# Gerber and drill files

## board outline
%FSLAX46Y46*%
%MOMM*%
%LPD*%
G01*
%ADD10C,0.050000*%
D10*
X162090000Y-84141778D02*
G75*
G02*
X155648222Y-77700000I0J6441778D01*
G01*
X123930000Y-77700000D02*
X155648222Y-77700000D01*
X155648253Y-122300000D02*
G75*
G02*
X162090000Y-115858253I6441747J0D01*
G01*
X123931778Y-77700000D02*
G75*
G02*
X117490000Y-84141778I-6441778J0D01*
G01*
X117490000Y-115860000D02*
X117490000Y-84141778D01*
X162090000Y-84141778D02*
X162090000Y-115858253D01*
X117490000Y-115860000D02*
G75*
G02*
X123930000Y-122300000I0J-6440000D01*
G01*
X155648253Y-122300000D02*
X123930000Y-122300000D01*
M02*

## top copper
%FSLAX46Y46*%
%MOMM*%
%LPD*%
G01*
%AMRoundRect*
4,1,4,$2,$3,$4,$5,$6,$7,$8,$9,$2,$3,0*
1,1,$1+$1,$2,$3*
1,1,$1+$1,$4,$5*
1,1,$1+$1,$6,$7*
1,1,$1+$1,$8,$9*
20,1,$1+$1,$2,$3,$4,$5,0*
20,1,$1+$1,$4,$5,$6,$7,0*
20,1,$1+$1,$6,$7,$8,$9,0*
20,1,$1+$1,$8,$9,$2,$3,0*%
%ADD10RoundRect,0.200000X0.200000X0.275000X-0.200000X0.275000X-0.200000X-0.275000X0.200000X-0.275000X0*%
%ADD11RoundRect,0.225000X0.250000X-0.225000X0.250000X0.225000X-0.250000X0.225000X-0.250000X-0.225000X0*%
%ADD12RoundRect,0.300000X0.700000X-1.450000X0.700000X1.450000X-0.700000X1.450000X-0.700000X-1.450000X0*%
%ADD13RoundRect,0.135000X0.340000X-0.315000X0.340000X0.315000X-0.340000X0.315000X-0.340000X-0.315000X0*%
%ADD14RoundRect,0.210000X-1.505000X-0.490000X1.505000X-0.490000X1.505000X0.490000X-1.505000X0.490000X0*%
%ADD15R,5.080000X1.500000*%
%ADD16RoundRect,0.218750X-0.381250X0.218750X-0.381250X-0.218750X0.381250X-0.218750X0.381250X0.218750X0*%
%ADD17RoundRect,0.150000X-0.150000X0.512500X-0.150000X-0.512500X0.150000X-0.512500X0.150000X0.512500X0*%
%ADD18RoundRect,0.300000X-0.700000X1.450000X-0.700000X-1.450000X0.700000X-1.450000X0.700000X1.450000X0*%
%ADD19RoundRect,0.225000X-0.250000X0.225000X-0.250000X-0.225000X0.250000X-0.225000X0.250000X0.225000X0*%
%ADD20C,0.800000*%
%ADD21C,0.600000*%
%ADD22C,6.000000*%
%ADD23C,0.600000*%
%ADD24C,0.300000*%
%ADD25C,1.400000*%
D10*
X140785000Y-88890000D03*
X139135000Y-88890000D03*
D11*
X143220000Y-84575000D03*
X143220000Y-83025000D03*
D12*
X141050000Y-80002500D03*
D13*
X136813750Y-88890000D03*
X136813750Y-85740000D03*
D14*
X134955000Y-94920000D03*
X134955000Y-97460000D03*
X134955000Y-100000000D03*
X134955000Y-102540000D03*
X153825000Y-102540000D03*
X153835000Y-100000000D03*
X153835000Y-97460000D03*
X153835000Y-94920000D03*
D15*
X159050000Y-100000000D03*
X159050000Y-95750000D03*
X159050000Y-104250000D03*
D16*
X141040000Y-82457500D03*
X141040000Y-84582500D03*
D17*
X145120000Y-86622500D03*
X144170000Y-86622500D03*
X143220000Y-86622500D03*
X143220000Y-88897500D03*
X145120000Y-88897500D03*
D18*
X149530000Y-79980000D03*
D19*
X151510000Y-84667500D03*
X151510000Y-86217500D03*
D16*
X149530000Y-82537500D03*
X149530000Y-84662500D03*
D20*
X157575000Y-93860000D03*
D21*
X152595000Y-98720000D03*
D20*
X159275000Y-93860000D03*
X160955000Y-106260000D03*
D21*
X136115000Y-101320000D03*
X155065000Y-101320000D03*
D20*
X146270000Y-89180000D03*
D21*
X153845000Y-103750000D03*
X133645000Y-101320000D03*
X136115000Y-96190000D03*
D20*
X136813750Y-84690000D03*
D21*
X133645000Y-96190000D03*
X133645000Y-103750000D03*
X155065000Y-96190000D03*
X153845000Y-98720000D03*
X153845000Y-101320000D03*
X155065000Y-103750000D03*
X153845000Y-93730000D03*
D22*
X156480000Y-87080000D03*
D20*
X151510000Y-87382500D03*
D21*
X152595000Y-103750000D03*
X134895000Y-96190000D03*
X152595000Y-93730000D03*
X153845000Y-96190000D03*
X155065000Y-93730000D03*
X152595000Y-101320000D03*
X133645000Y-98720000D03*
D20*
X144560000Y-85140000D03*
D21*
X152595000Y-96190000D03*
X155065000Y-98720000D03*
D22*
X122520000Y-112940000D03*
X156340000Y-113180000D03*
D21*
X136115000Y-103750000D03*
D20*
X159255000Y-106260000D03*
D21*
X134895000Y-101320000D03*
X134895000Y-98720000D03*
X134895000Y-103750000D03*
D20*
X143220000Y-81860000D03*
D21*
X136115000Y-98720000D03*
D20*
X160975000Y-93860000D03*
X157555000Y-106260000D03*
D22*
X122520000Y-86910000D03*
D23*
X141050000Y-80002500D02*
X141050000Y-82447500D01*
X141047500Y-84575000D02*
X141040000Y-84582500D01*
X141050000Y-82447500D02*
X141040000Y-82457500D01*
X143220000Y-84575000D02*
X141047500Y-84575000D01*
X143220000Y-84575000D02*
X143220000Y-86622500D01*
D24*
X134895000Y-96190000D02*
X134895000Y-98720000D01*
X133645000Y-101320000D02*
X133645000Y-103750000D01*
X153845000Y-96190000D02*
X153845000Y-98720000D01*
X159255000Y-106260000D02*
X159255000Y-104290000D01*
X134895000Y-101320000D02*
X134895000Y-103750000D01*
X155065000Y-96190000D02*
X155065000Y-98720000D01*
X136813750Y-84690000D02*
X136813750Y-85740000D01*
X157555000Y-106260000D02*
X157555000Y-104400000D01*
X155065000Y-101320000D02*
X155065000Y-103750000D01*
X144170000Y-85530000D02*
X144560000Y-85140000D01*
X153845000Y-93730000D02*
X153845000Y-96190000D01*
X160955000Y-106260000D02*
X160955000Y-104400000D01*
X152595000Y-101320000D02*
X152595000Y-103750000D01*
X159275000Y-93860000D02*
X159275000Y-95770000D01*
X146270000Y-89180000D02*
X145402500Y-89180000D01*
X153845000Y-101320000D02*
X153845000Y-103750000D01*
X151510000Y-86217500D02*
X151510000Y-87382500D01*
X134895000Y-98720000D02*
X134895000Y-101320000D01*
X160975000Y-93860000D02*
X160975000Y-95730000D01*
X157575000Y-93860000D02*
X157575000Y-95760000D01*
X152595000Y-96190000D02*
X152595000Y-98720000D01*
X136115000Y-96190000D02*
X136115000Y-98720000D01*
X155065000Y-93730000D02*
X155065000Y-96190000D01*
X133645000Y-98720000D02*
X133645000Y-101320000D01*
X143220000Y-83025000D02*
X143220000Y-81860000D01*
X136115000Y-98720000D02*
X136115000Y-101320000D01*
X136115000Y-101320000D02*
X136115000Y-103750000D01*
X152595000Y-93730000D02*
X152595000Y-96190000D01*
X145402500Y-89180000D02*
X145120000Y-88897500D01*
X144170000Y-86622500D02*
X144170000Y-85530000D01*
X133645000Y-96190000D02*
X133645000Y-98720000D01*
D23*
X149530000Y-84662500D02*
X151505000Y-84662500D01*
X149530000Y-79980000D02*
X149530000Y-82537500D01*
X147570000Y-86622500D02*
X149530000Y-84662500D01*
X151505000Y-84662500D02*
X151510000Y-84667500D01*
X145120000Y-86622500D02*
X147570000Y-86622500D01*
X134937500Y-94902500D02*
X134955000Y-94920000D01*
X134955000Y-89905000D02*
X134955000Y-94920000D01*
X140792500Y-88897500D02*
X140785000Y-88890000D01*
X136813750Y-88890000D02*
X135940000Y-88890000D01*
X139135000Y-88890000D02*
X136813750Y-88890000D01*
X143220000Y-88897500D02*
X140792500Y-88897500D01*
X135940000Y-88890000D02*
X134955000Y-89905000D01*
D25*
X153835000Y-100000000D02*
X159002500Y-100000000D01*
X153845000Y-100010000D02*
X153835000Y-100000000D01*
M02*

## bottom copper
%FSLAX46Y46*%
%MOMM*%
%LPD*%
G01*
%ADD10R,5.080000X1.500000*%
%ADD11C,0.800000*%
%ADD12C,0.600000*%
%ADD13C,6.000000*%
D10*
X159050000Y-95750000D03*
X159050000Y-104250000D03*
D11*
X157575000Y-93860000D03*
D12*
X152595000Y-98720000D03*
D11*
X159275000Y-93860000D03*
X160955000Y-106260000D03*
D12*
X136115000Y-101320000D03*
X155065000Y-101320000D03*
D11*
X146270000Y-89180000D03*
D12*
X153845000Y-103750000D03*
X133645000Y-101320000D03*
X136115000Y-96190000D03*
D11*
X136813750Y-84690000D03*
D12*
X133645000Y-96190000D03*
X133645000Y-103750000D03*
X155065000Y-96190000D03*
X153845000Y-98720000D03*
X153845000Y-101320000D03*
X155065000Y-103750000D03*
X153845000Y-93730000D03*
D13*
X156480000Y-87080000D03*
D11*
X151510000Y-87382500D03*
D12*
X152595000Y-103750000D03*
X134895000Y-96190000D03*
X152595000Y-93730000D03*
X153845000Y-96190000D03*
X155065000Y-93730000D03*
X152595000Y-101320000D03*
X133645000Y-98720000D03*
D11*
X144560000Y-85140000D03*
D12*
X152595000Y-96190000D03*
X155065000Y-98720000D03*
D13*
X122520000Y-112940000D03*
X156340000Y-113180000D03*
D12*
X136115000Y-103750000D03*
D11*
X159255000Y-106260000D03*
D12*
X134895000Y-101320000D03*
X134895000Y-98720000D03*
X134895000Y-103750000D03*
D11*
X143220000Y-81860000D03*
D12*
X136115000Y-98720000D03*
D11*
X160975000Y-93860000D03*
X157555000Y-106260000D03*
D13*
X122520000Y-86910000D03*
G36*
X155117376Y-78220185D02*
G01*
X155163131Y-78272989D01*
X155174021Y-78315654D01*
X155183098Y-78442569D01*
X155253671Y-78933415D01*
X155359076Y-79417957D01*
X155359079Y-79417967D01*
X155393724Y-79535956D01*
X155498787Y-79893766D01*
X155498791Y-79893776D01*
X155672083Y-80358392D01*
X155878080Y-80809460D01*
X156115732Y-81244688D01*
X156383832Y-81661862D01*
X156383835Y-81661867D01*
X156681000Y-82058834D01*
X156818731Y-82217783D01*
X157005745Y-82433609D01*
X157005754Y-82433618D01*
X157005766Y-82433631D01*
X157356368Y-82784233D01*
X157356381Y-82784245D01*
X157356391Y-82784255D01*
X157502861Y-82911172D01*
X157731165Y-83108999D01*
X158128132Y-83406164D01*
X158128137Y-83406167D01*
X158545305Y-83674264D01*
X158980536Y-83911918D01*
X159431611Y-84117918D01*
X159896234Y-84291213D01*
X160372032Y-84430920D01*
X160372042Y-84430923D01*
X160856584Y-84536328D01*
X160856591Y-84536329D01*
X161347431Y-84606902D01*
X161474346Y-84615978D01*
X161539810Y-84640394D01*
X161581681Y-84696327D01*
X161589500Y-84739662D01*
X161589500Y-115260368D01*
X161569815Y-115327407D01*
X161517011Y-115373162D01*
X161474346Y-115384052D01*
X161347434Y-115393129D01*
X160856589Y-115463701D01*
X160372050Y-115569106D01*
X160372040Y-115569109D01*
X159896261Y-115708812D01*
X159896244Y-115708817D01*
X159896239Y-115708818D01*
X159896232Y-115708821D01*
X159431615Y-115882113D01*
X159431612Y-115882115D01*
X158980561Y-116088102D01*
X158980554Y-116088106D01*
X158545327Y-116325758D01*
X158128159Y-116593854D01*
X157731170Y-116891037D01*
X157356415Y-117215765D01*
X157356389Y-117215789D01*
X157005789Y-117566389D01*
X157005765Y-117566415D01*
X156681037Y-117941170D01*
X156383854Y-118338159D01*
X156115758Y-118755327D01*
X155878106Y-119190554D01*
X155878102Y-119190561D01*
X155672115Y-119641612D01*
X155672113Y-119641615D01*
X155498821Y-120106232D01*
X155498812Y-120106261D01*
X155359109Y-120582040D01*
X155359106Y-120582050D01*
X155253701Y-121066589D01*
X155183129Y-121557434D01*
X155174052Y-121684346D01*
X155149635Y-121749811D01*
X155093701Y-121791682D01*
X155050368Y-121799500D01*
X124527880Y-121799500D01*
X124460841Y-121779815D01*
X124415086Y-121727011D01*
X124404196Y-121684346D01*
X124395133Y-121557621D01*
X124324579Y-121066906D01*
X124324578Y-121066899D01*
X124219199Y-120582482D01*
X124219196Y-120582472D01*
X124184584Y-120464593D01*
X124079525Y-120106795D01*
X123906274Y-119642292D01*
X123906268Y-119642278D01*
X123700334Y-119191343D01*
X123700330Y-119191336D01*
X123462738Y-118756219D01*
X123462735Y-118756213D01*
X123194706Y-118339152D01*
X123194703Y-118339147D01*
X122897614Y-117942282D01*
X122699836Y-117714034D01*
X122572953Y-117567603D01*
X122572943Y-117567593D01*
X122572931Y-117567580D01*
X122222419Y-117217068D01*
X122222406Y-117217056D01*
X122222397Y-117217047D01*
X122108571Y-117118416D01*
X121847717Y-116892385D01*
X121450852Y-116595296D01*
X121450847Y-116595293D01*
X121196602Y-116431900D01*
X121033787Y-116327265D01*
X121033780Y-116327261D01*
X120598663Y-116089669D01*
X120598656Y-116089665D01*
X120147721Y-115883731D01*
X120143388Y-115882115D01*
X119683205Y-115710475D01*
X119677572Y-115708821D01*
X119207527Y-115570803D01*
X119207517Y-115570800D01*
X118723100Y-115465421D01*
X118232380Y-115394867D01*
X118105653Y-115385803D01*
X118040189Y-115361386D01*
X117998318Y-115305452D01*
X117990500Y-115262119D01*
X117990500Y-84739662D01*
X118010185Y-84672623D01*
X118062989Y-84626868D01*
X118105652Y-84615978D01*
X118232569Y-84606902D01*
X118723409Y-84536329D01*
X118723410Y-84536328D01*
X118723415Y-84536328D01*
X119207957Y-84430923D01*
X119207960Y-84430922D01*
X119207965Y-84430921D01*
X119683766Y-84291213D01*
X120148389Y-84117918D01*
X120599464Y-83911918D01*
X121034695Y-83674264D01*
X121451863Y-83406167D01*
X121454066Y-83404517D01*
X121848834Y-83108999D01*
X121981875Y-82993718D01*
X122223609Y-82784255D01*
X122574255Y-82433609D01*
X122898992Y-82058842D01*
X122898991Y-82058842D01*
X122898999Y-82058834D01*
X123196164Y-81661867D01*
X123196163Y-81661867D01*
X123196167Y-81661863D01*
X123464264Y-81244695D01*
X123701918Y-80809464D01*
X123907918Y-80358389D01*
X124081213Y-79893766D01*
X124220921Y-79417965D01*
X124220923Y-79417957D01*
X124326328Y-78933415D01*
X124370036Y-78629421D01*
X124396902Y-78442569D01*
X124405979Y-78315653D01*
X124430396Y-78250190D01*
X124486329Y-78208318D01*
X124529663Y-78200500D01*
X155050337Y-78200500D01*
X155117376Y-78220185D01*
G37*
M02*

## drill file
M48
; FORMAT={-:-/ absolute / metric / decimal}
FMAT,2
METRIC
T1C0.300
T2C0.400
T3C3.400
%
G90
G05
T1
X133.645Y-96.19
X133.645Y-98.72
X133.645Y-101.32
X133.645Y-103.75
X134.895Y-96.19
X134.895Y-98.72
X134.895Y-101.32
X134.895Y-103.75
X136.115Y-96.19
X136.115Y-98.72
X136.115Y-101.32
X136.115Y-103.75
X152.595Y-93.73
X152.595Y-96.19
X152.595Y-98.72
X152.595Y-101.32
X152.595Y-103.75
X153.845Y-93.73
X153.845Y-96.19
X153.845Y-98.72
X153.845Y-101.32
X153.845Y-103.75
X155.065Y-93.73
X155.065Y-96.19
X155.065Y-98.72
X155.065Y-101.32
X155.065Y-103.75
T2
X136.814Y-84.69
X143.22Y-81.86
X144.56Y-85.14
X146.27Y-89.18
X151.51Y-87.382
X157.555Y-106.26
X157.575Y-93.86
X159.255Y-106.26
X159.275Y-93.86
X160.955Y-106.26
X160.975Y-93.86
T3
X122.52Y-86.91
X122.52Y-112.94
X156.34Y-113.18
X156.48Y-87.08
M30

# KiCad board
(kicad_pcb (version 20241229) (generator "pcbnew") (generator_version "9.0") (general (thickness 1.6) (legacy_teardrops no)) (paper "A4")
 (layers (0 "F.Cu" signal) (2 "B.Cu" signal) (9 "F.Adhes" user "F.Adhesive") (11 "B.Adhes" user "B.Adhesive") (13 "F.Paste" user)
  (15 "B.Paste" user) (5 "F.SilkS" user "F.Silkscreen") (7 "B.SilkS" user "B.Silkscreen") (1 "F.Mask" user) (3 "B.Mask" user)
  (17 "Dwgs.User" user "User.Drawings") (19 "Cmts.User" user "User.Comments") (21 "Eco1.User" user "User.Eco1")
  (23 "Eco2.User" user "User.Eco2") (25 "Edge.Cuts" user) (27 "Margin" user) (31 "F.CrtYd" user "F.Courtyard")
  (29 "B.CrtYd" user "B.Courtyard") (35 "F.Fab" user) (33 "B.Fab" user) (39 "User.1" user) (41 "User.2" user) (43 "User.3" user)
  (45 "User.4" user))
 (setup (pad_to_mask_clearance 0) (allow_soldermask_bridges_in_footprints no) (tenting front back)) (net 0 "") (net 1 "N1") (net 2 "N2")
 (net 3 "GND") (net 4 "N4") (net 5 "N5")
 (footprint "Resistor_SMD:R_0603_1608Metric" (layer "F.Cu") (at 139.96 88.89 180)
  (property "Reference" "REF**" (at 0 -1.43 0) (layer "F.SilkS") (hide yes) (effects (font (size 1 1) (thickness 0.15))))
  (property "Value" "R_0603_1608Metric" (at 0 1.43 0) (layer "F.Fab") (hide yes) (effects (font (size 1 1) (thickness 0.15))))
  (pad "1" smd roundrect (at -0.825 0 180) (size 0.8 0.95) (layers "F.Cu" "F.Mask" "F.Paste") (roundrect_rratio 0.25) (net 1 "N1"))
  (pad "2" smd roundrect (at 0.825 0 180) (size 0.8 0.95) (layers "F.Cu" "F.Mask" "F.Paste") (roundrect_rratio 0.25) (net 1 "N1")))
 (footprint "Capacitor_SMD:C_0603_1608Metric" (layer "F.Cu") (at 143.22 83.8 90)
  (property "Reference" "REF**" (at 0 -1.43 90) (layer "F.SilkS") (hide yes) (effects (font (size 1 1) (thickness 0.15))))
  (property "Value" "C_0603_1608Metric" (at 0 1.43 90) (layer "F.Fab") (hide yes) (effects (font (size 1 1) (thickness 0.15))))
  (pad "1" smd roundrect (at -0.775 0 90) (size 0.9 0.95) (layers "F.Cu" "F.Mask" "F.Paste") (roundrect_rratio 0.25) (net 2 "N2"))
  (pad "2" smd roundrect (at 0.775 0 90) (size 0.9 0.95) (layers "F.Cu" "F.Mask" "F.Paste") (roundrect_rratio 0.25) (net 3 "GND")))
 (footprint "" (layer "F.Cu") (at 141.05 80.0125 180)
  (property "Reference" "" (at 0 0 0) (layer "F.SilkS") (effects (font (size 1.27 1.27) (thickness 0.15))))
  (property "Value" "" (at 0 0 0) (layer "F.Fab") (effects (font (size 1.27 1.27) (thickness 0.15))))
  (pad "3" smd roundrect (at 0 0.01 90) (size 3.5 2) (layers "F.Cu" "F.Mask" "F.Paste") (roundrect_rratio 0.15) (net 2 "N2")
   (thermal_bridge_angle 45)))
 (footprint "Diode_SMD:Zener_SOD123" (layer "F.Cu") (at 136.80375 88.89 90)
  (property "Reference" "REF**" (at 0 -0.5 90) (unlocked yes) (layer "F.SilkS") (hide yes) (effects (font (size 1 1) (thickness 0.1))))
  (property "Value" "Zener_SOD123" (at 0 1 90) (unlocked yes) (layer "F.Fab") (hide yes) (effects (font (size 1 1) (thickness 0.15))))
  (pad "1" smd roundrect (at 0 0.01 90) (size 0.9 0.95) (layers "F.Cu" "F.Mask" "F.Paste") (roundrect_rratio 0.15) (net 1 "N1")
   (thermal_bridge_angle 45))
  (pad "2" smd roundrect (at 3.15 0.01 90) (size 0.9 0.95) (layers "F.Cu" "F.Mask" "F.Paste") (roundrect_rratio 0.15) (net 3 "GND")
   (thermal_bridge_angle 45)))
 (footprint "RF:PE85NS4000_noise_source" (layer "F.Cu") (at 144.395 98.73)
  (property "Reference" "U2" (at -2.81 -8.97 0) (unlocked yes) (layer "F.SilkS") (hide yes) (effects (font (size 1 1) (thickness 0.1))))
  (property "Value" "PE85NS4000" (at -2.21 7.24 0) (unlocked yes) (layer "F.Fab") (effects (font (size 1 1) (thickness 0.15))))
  (pad "1" smd roundrect (at -9.44 -3.81) (size 3.43 1.4) (layers "F.Cu" "F.Mask" "F.Paste") (roundrect_rratio 0.15) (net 1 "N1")
   (thermal_bridge_angle 45))
  (pad "2" smd roundrect (at -9.44 -1.27) (size 3.43 1.4) (layers "F.Cu" "F.Mask" "F.Paste") (roundrect_rratio 0.15) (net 3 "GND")
   (thermal_bridge_angle 45))
  (pad "3" smd roundrect (at -9.44 1.27) (size 3.43 1.4) (layers "F.Cu" "F.Mask" "F.Paste") (roundrect_rratio 0.15) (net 3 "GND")
   (thermal_bridge_angle 45))
  (pad "4" smd roundrect (at -9.44 3.81) (size 3.43 1.4) (layers "F.Cu" "F.Mask" "F.Paste") (roundrect_rratio 0.15) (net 3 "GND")
   (thermal_bridge_angle 45))
  (pad "5" smd roundrect (at 9.43 3.81) (size 3.43 1.4) (layers "F.Cu" "F.Mask" "F.Paste") (roundrect_rratio 0.15) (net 3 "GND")
   (thermal_bridge_angle 45))
  (pad "6" smd roundrect (at 9.44 1.27) (size 3.43 1.4) (layers "F.Cu" "F.Mask" "F.Paste") (roundrect_rratio 0.15) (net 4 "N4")
   (thermal_bridge_angle 45))
  (pad "7" smd roundrect (at 9.44 -1.27) (size 3.43 1.4) (layers "F.Cu" "F.Mask" "F.Paste") (roundrect_rratio 0.15) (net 3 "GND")
   (thermal_bridge_angle 45))
  (pad "8" smd roundrect (at 9.44 -3.81) (size 3.43 1.4) (layers "F.Cu" "F.Mask" "F.Paste") (roundrect_rratio 0.15) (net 3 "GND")
   (thermal_bridge_angle 45)))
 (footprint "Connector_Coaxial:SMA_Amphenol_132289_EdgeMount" (layer "F.Cu") (at 159.05 100)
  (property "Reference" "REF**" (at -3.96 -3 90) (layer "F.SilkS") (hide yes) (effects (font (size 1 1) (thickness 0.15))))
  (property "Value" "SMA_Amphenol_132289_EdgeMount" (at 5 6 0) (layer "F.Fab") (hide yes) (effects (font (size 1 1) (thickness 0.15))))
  (pad "1" smd rect (at 0 0 90) (size 1.5 5.08) (layers "F.Cu" "F.Mask" "F.Paste") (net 4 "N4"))
  (pad "2" smd rect (at 0 -4.25 90) (size 1.5 5.08) (layers "F.Cu" "F.Mask" "F.Paste") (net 3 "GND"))
  (pad "2" smd rect (at 0 -4.25 90) (size 1.5 5.08) (layers "B.Cu" "B.Mask" "B.Paste") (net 3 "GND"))
  (pad "2" smd rect (at 0 4.25 90) (size 1.5 5.08) (layers "F.Cu" "F.Mask" "F.Paste") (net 3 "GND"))
  (pad "2" smd rect (at 0 4.25 90) (size 1.5 5.08) (layers "B.Cu" "B.Mask" "B.Paste") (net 3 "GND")))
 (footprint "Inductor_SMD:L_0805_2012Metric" (layer "F.Cu") (at 141.04 83.52 -90)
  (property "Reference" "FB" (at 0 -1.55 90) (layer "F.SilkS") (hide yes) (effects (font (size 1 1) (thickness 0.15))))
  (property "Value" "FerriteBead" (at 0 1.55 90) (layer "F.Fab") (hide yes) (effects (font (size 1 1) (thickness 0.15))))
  (pad "1" smd roundrect (at -1.0625 0 270) (size 0.875 1.2) (layers "F.Cu" "F.Mask" "F.Paste") (roundrect_rratio 0.25) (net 2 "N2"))
  (pad "2" smd roundrect (at 1.0625 0 270) (size 0.875 1.2) (layers "F.Cu" "F.Mask" "F.Paste") (roundrect_rratio 0.25) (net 2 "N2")))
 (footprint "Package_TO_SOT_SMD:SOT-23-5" (layer "F.Cu") (at 144.17 87.76 -90)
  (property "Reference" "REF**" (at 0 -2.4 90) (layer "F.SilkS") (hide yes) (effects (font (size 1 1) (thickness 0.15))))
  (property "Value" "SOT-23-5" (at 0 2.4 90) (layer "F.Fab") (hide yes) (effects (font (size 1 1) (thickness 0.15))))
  (pad "1" smd roundrect (at -1.1375 -0.95 270) (size 1.325 0.6) (layers "F.Cu" "F.Mask" "F.Paste") (roundrect_rratio 0.25) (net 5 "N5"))
  (pad "2" smd roundrect (at -1.1375 0 270) (size 1.325 0.6) (layers "F.Cu" "F.Mask" "F.Paste") (roundrect_rratio 0.25) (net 3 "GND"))
  (pad "3" smd roundrect (at -1.1375 0.95 270) (size 1.325 0.6) (layers "F.Cu" "F.Mask" "F.Paste") (roundrect_rratio 0.25) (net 2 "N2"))
  (pad "4" smd roundrect (at 1.1375 0.95 270) (size 1.325 0.6) (layers "F.Cu" "F.Mask" "F.Paste") (roundrect_rratio 0.25) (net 1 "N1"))
  (pad "5" smd roundrect (at 1.1375 -0.95 270) (size 1.325 0.6) (layers "F.Cu" "F.Mask" "F.Paste") (roundrect_rratio 0.25) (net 3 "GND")))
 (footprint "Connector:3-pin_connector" (layer "F.Cu") (at 149.53 79.98 -90)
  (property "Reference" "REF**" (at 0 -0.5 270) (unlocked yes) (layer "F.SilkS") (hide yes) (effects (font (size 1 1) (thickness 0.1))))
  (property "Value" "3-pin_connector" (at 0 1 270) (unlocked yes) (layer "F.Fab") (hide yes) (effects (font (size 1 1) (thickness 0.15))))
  (pad "1" smd roundrect (at 0 0 270) (size 3.5 2) (layers "F.Cu" "F.Mask" "F.Paste") (roundrect_rratio 0.15) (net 5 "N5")
   (thermal_bridge_angle 45)))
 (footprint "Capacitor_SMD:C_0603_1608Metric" (layer "F.Cu") (at 151.51 85.4425 -90)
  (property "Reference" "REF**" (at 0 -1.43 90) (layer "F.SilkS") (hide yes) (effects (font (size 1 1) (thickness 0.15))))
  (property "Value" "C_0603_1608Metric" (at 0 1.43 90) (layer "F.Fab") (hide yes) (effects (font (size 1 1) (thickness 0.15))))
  (pad "1" smd roundrect (at -0.775 0 270) (size 0.9 0.95) (layers "F.Cu" "F.Mask" "F.Paste") (roundrect_rratio 0.25) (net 5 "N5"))
  (pad "2" smd roundrect (at 0.775 0 270) (size 0.9 0.95) (layers "F.Cu" "F.Mask" "F.Paste") (roundrect_rratio 0.25) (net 3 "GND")))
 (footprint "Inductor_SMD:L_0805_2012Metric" (layer "F.Cu") (at 149.53 83.6 -90)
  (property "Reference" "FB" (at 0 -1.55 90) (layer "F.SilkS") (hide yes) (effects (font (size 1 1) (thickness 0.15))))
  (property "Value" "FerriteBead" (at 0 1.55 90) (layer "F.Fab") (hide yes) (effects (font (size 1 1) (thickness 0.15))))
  (pad "1" smd roundrect (at -1.0625 0 270) (size 0.875 1.2) (layers "F.Cu" "F.Mask" "F.Paste") (roundrect_rratio 0.25) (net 5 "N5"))
  (pad "2" smd roundrect (at 1.0625 0 270) (size 0.875 1.2) (layers "F.Cu" "F.Mask" "F.Paste") (roundrect_rratio 0.25) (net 5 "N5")))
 (gr_arc (start 162.09 84.141778) (mid 157.534975 82.255025) (end 155.648222 77.7) (stroke (width 0.05) (type default)) (layer "Edge.Cuts"))
 (gr_line (start 123.93 77.7) (end 155.648222 77.7) (stroke (width 0.05) (type default)) (layer "Edge.Cuts"))
 (gr_arc (start 155.648253 122.3) (mid 157.534997 117.744997) (end 162.09 115.858253) (stroke (width 0.05) (type default))
  (layer "Edge.Cuts"))
 (gr_arc (start 123.931778 77.7) (mid 122.045025 82.255025) (end 117.49 84.141778) (stroke (width 0.05) (type default)) (layer "Edge.Cuts"))
 (gr_line (start 117.49 115.86) (end 117.49 84.141778) (stroke (width 0.05) (type default)) (layer "Edge.Cuts"))
 (gr_line (start 162.09 84.141778) (end 162.09 115.858253) (stroke (width 0.05) (type default)) (layer "Edge.Cuts"))
 (gr_arc (start 117.49 115.86) (mid 122.043768 117.746232) (end 123.93 122.3) (stroke (width 0.05) (type default)) (layer "Edge.Cuts"))
 (gr_line (start 155.648253 122.3) (end 123.93 122.3) (stroke (width 0.05) (type default)) (layer "Edge.Cuts"))
 (segment (start 141.05 80.0025) (end 141.05 82.4475) (width 0.6) (layer "F.Cu") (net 2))
 (segment (start 141.0475 84.575) (end 141.04 84.5825) (width 0.6) (layer "F.Cu") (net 2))
 (segment (start 141.05 82.4475) (end 141.04 82.4575) (width 0.6) (layer "F.Cu") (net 2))
 (segment (start 143.22 84.575) (end 141.0475 84.575) (width 0.6) (layer "F.Cu") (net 2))
 (segment (start 143.22 84.575) (end 143.22 86.6225) (width 0.6) (layer "F.Cu") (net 2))
 (segment (start 134.895 96.19) (end 134.895 98.72) (width 0.3) (layer "F.Cu") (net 3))
 (segment (start 133.645 101.32) (end 133.645 103.75) (width 0.3) (layer "F.Cu") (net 3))
 (segment (start 153.845 96.19) (end 153.845 98.72) (width 0.3) (layer "F.Cu") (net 3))
 (segment (start 159.255 106.26) (end 159.255 104.29) (width 0.3) (layer "F.Cu") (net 3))
 (segment (start 134.895 101.32) (end 134.895 103.75) (width 0.3) (layer "F.Cu") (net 3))
 (segment (start 155.065 96.19) (end 155.065 98.72) (width 0.3) (layer "F.Cu") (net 3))
 (segment (start 136.81375 84.69) (end 136.81375 85.74) (width 0.3) (layer "F.Cu") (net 3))
 (segment (start 157.555 106.26) (end 157.555 104.4) (width 0.3) (layer "F.Cu") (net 3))
 (segment (start 155.065 101.32) (end 155.065 103.75) (width 0.3) (layer "F.Cu") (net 3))
 (segment (start 144.17 85.53) (end 144.56 85.14) (width 0.3) (layer "F.Cu") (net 3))
 (segment (start 153.845 93.73) (end 153.845 96.19) (width 0.3) (layer "F.Cu") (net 3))
 (segment (start 160.955 106.26) (end 160.955 104.4) (width 0.3) (layer "F.Cu") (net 3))
 (segment (start 152.595 101.32) (end 152.595 103.75) (width 0.3) (layer "F.Cu") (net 3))
 (segment (start 159.275 93.86) (end 159.275 95.77) (width 0.3) (layer "F.Cu") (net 3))
 (segment (start 146.27 89.18) (end 145.4025 89.18) (width 0.3) (layer "F.Cu") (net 3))
 (segment (start 153.845 101.32) (end 153.845 103.75) (width 0.3) (layer "F.Cu") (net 3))
 (segment (start 151.51 86.2175) (end 151.51 87.3825) (width 0.3) (layer "F.Cu") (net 3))
 (segment (start 134.895 98.72) (end 134.895 101.32) (width 0.3) (layer "F.Cu") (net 3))
 (segment (start 160.975 93.86) (end 160.975 95.73) (width 0.3) (layer "F.Cu") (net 3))
 (segment (start 157.575 93.86) (end 157.575 95.76) (width 0.3) (layer "F.Cu") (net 3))
 (segment (start 152.595 96.19) (end 152.595 98.72) (width 0.3) (layer "F.Cu") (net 3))
 (segment (start 136.115 96.19) (end 136.115 98.72) (width 0.3) (layer "F.Cu") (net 3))
 (segment (start 155.065 93.73) (end 155.065 96.19) (width 0.3) (layer "F.Cu") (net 3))
 (segment (start 133.645 98.72) (end 133.645 101.32) (width 0.3) (layer "F.Cu") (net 3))
 (segment (start 143.22 83.025) (end 143.22 81.86) (width 0.3) (layer "F.Cu") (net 3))
 (segment (start 136.115 98.72) (end 136.115 101.32) (width 0.3) (layer "F.Cu") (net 3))
 (segment (start 136.115 101.32) (end 136.115 103.75) (width 0.3) (layer "F.Cu") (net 3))
 (segment (start 152.595 93.73) (end 152.595 96.19) (width 0.3) (layer "F.Cu") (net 3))
 (segment (start 145.4025 89.18) (end 145.12 88.8975) (width 0.3) (layer "F.Cu") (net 3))
 (segment (start 144.17 86.6225) (end 144.17 85.53) (width 0.3) (layer "F.Cu") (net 3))
 (segment (start 133.645 96.19) (end 133.645 98.72) (width 0.3) (layer "F.Cu") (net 3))
 (via (at 157.575 93.86) (size 0.8) (drill 0.4) (layers "F.Cu" "B.Cu") (free yes) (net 3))
 (via (at 152.595 98.72) (size 0.6) (drill 0.3) (layers "F.Cu" "B.Cu") (free yes) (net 3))
 (via (at 159.275 93.86) (size 0.8) (drill 0.4) (layers "F.Cu" "B.Cu") (free yes) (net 3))
 (via (at 160.955 106.26) (size 0.8) (drill 0.4) (layers "F.Cu" "B.Cu") (free yes) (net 3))
 (via (at 136.115 101.32) (size 0.6) (drill 0.3) (layers "F.Cu" "B.Cu") (free yes) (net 3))
 (via (at 155.065 101.32) (size 0.6) (drill 0.3) (layers "F.Cu" "B.Cu") (free yes) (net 3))
 (via (at 146.27 89.18) (size 0.8) (drill 0.4) (layers "F.Cu" "B.Cu") (free yes) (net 3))
 (via (at 153.845 103.75) (size 0.6) (drill 0.3) (layers "F.Cu" "B.Cu") (free yes) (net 3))
 (via (at 133.645 101.32) (size 0.6) (drill 0.3) (layers "F.Cu" "B.Cu") (free yes) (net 3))
 (via (at 136.115 96.19) (size 0.6) (drill 0.3) (layers "F.Cu" "B.Cu") (free yes) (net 3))
 (via (at 136.81375 84.69) (size 0.8) (drill 0.4) (layers "F.Cu" "B.Cu") (free yes) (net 3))
 (via (at 133.645 96.19) (size 0.6) (drill 0.3) (layers "F.Cu" "B.Cu") (free yes) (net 3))
 (via (at 133.645 103.75) (size 0.6) (drill 0.3) (layers "F.Cu" "B.Cu") (free yes) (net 3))
 (via (at 155.065 96.19) (size 0.6) (drill 0.3) (layers "F.Cu" "B.Cu") (free yes) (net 3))
 (via (at 153.845 98.72) (size 0.6) (drill 0.3) (layers "F.Cu" "B.Cu") (free yes) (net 3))
 (via (at 153.845 101.32) (size 0.6) (drill 0.3) (layers "F.Cu" "B.Cu") (free yes) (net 3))
 (via (at 155.065 103.75) (size 0.6) (drill 0.3) (layers "F.Cu" "B.Cu") (free yes) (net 3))
 (via (at 153.845 93.73) (size 0.6) (drill 0.3) (layers "F.Cu" "B.Cu") (free yes) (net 3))
 (via (at 156.48 87.08) (size 6) (drill 3.4) (layers "F.Cu" "B.Cu") (free yes) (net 3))
 (via (at 151.51 87.3825) (size 0.8) (drill 0.4) (layers "F.Cu" "B.Cu") (free yes) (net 3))
 (via (at 152.595 103.75) (size 0.6) (drill 0.3) (layers "F.Cu" "B.Cu") (free yes) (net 3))
 (via (at 134.895 96.19) (size 0.6) (drill 0.3) (layers "F.Cu" "B.Cu") (free yes) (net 3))
 (via (at 152.595 93.73) (size 0.6) (drill 0.3) (layers "F.Cu" "B.Cu") (free yes) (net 3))
 (via (at 153.845 96.19) (size 0.6) (drill 0.3) (layers "F.Cu" "B.Cu") (free yes) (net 3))
 (via (at 155.065 93.73) (size 0.6) (drill 0.3) (layers "F.Cu" "B.Cu") (free yes) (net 3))
 (via (at 152.595 101.32) (size 0.6) (drill 0.3) (layers "F.Cu" "B.Cu") (free yes) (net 3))
 (via (at 133.645 98.72) (size 0.6) (drill 0.3) (layers "F.Cu" "B.Cu") (free yes) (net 3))
 (via (at 144.56 85.14) (size 0.8) (drill 0.4) (layers "F.Cu" "B.Cu") (free yes) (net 3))
 (via (at 152.595 96.19) (size 0.6) (drill 0.3) (layers "F.Cu" "B.Cu") (free yes) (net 3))
 (via (at 155.065 98.72) (size 0.6) (drill 0.3) (layers "F.Cu" "B.Cu") (free yes) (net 3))
 (via (at 122.52 112.94) (size 6) (drill 3.4) (layers "F.Cu" "B.Cu") (free yes) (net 3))
 (via (at 156.34 113.18) (size 6) (drill 3.4) (layers "F.Cu" "B.Cu") (free yes) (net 3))
 (via (at 136.115 103.75) (size 0.6) (drill 0.3) (layers "F.Cu" "B.Cu") (free yes) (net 3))
 (via (at 159.255 106.26) (size 0.8) (drill 0.4) (layers "F.Cu" "B.Cu") (free yes) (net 3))
 (via (at 134.895 101.32) (size 0.6) (drill 0.3) (layers "F.Cu" "B.Cu") (free yes) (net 3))
 (via (at 134.895 98.72) (size 0.6) (drill 0.3) (layers "F.Cu" "B.Cu") (free yes) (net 3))
 (via (at 134.895 103.75) (size 0.6) (drill 0.3) (layers "F.Cu" "B.Cu") (free yes) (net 3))
 (via (at 143.22 81.86) (size 0.8) (drill 0.4) (layers "F.Cu" "B.Cu") (free yes) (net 3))
 (via (at 136.115 98.72) (size 0.6) (drill 0.3) (layers "F.Cu" "B.Cu") (free yes) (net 3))
 (via (at 160.975 93.86) (size 0.8) (drill 0.4) (layers "F.Cu" "B.Cu") (free yes) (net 3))
 (via (at 157.555 106.26) (size 0.8) (drill 0.4) (layers "F.Cu" "B.Cu") (free yes) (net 3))
 (via (at 122.52 86.91) (size 6) (drill 3.4) (layers "F.Cu" "B.Cu") (free yes) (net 3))
 (segment (start 149.53 84.6625) (end 151.505 84.6625) (width 0.6) (layer "F.Cu") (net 5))
 (segment (start 149.53 79.98) (end 149.53 82.5375) (width 0.6) (layer "F.Cu") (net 5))
 (segment (start 147.57 86.6225) (end 149.53 84.6625) (width 0.6) (layer "F.Cu") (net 5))
 (segment (start 151.505 84.6625) (end 151.51 84.6675) (width 0.6) (layer "F.Cu") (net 5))
 (segment (start 145.12 86.6225) (end 147.57 86.6225) (width 0.6) (layer "F.Cu") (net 5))
 (segment (start 134.9375 94.9025) (end 134.955 94.92) (width 0.6) (layer "F.Cu") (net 1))
 (segment (start 134.955 89.905) (end 134.955 94.92) (width 0.6) (layer "F.Cu") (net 1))
 (segment (start 140.7925 88.8975) (end 140.785 88.89) (width 0.6) (layer "F.Cu") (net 1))
 (segment (start 136.81375 88.89) (end 135.94 88.89) (width 0.6) (layer "F.Cu") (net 1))
 (segment (start 139.135 88.89) (end 136.81375 88.89) (width 0.6) (layer "F.Cu") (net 1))
 (segment (start 143.22 88.8975) (end 140.7925 88.8975) (width 0.6) (layer "F.Cu") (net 1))
 (segment (start 135.94 88.89) (end 134.955 89.905) (width 0.6) (layer "F.Cu") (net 1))
 (segment (start 153.835 100) (end 159.0025 100) (width 1.4) (layer "F.Cu") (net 4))
 (segment (start 153.845 100.01) (end 153.835 100) (width 1.4) (layer "F.Cu") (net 4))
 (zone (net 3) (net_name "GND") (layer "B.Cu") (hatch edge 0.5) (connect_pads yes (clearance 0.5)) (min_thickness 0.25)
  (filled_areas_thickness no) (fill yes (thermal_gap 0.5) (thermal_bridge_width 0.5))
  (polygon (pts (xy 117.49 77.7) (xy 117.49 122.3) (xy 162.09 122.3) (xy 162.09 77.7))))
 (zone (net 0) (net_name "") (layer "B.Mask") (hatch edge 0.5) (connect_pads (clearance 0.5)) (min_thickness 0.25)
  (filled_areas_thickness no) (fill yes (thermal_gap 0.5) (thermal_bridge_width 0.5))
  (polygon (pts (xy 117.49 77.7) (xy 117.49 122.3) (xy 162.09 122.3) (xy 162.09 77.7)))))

